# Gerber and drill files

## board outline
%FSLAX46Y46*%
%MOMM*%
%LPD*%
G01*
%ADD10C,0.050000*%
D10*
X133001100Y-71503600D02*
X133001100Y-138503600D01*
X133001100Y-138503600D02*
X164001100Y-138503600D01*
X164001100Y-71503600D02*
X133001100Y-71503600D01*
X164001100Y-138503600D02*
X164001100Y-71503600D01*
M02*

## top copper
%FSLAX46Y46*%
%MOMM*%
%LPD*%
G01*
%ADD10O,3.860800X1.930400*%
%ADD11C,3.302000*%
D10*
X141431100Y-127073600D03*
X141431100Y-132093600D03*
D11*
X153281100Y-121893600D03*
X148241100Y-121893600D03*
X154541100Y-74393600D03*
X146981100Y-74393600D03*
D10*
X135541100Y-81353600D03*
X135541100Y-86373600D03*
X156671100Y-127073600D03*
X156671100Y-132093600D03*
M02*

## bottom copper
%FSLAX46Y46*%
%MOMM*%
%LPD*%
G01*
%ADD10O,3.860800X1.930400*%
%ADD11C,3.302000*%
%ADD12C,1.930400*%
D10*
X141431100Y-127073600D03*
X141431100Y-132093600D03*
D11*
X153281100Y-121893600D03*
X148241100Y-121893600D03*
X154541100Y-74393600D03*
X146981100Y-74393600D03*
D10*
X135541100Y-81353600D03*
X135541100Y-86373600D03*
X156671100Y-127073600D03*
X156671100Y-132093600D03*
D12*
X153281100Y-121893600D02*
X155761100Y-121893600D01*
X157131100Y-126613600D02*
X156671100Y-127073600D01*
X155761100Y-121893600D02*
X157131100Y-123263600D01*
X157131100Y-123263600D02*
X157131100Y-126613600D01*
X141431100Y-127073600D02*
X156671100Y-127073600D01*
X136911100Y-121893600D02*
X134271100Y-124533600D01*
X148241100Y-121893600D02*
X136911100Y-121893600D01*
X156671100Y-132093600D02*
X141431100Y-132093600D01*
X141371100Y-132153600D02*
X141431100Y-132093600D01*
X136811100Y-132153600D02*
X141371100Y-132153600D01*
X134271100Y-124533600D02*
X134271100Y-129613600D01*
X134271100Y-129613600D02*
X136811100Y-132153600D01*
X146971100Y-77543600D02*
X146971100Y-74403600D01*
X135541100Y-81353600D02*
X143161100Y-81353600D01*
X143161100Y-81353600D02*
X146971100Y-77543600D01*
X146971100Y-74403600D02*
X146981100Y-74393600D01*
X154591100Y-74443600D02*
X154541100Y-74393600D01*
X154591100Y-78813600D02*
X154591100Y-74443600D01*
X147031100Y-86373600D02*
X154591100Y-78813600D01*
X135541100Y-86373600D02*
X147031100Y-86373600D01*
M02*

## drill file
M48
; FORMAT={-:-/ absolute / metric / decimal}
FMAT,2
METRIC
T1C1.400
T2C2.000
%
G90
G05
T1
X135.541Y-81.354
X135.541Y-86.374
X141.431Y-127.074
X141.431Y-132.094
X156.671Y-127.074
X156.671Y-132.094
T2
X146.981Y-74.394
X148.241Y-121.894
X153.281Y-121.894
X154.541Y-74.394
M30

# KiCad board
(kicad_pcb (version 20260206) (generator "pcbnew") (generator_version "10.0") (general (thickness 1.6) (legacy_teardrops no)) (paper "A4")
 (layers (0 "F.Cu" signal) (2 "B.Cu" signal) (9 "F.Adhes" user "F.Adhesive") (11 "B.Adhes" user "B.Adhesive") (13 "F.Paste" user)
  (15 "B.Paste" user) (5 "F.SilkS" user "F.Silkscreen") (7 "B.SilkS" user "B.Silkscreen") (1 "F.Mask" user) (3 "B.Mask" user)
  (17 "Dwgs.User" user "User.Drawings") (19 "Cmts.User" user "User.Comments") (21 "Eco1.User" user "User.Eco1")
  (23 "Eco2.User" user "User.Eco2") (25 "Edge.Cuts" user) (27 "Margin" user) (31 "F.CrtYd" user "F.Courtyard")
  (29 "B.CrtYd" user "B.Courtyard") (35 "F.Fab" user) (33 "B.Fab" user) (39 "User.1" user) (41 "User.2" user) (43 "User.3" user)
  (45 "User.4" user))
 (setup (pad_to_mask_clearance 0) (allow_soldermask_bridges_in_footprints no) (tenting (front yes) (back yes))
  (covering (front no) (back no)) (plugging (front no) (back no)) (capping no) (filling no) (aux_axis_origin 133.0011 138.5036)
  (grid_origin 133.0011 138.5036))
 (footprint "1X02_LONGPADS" (layer "F.Cu") (at 141.4311 127.0736 -90)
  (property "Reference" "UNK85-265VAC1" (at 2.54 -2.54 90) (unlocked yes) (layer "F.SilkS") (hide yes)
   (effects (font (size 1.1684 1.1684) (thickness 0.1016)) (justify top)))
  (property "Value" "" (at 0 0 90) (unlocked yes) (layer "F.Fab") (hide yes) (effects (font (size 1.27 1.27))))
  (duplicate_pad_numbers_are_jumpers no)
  (pad "1" thru_hole oval (at 0 0) (size 3.8608 1.9304) (drill 1.4) (layers "*.Cu" "*.Mask") (remove_unused_layers no) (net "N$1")
   (solder_mask_margin 0.1016) (thermal_bridge_angle 0))
  (pad "2" thru_hole oval (at 5.02 0) (size 3.8608 1.9304) (drill 1.4) (layers "*.Cu" "*.Mask") (remove_unused_layers no) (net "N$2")
   (solder_mask_margin 0.1016) (thermal_bridge_angle 0)))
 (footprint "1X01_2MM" (layer "F.Cu") (at 153.2811 121.8936)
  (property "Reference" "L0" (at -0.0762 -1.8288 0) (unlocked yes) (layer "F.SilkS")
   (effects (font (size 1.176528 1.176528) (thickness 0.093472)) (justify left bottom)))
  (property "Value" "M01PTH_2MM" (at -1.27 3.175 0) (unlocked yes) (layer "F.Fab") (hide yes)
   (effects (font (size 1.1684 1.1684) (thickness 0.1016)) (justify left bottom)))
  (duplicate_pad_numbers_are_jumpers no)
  (pad "1" thru_hole circle (at 0 0 90) (size 3.302 3.302) (drill 2) (layers "*.Cu" "*.Mask") (remove_unused_layers no) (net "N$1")
   (solder_mask_margin 0.1016) (thermal_bridge_angle 0)))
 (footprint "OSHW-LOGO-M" (layer "F.Cu") (at 135.5411 75.0036 90)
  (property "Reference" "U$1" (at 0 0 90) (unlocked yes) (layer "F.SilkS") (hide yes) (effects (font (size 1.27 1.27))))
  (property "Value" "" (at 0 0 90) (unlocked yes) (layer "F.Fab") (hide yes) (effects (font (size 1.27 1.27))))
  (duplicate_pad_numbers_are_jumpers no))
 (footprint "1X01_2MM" (layer "F.Cu") (at 148.2411 121.8936)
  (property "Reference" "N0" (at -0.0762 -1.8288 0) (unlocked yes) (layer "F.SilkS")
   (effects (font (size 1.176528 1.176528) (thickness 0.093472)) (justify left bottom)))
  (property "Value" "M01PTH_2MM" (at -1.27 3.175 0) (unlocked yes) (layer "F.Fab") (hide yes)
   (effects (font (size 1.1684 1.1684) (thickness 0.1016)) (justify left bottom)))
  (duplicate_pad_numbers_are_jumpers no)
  (pad "1" thru_hole circle (at 0 0 90) (size 3.302 3.302) (drill 2) (layers "*.Cu" "*.Mask") (remove_unused_layers no) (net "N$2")
   (solder_mask_margin 0.1016) (thermal_bridge_angle 0)))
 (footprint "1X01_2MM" (layer "F.Cu") (at 154.5411 74.3936)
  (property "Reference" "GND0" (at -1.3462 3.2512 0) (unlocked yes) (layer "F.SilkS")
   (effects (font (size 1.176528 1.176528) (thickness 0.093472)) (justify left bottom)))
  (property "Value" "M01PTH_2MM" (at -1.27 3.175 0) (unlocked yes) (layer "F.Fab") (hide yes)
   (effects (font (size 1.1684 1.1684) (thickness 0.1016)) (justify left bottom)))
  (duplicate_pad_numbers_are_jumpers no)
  (pad "1" thru_hole circle (at 0 0 90) (size 3.302 3.302) (drill 2) (layers "*.Cu" "*.Mask") (remove_unused_layers no) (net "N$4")
   (solder_mask_margin 0.1016) (thermal_bridge_angle 0)))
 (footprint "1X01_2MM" (layer "F.Cu") (at 146.9811 74.3936)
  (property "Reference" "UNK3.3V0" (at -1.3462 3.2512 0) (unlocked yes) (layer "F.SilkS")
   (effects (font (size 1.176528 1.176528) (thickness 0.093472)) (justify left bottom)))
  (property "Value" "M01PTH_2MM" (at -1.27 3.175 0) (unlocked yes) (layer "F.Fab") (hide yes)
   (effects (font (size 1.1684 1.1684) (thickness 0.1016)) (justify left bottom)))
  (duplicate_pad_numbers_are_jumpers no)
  (pad "1" thru_hole circle (at 0 0 90) (size 3.302 3.302) (drill 2) (layers "*.Cu" "*.Mask") (remove_unused_layers no) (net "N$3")
   (solder_mask_margin 0.1016) (thermal_bridge_angle 0)))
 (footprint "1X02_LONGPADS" (layer "F.Cu") (at 135.5411 81.3536 -90)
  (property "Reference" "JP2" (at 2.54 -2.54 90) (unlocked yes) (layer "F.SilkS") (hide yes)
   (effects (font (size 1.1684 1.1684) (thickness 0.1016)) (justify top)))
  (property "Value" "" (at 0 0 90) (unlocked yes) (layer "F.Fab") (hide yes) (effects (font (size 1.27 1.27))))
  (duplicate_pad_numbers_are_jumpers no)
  (pad "1" thru_hole oval (at 0 0) (size 3.8608 1.9304) (drill 1.4) (layers "*.Cu" "*.Mask") (remove_unused_layers no) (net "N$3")
   (solder_mask_margin 0.1016) (thermal_bridge_angle 0))
  (pad "2" thru_hole oval (at 5.02 0) (size 3.8608 1.9304) (drill 1.4) (layers "*.Cu" "*.Mask") (remove_unused_layers no) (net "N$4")
   (solder_mask_margin 0.1016) (thermal_bridge_angle 0)))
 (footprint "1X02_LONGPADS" (layer "F.Cu") (at 156.6711 127.0736 -90)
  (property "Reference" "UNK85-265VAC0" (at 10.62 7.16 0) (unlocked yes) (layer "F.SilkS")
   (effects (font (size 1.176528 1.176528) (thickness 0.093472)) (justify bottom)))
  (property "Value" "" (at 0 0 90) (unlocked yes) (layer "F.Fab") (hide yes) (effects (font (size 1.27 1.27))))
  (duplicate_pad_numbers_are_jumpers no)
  (pad "1" thru_hole oval (at 0 0) (size 3.8608 1.9304) (drill 1.4) (layers "*.Cu" "*.Mask") (remove_unused_layers no) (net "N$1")
   (solder_mask_margin 0.1016) (thermal_bridge_angle 0))
  (pad "2" thru_hole oval (at 5.02 0) (size 3.8608 1.9304) (drill 1.4) (layers "*.Cu" "*.Mask") (remove_unused_layers no) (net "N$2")
   (solder_mask_margin 0.1016) (thermal_bridge_angle 0)))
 (gr_line (start 133.0011 71.5036) (end 133.0011 138.5036) (stroke (width 0.05) (type solid)) (layer "Edge.Cuts"))
 (gr_line (start 133.0011 138.5036) (end 164.0011 138.5036) (stroke (width 0.05) (type solid)) (layer "Edge.Cuts"))
 (gr_line (start 164.0011 71.5036) (end 133.0011 71.5036) (stroke (width 0.05) (type solid)) (layer "Edge.Cuts"))
 (gr_line (start 164.0011 138.5036) (end 164.0011 71.5036) (stroke (width 0.05) (type solid)) (layer "Edge.Cuts"))
 (segment (start 153.2811 121.8936) (end 155.7611 121.8936) (width 1.9304) (layer "B.Cu") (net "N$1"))
 (segment (start 157.1311 126.6136) (end 156.6711 127.0736) (width 1.9304) (layer "B.Cu") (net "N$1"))
 (segment (start 155.7611 121.8936) (end 157.1311 123.2636) (width 1.9304) (layer "B.Cu") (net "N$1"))
 (segment (start 157.1311 123.2636) (end 157.1311 126.6136) (width 1.9304) (layer "B.Cu") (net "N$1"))
 (segment (start 141.4311 127.0736) (end 156.6711 127.0736) (width 1.9304) (layer "B.Cu") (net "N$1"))
 (segment (start 136.9111 121.8936) (end 134.2711 124.5336) (width 1.9304) (layer "B.Cu") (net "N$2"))
 (segment (start 148.2411 121.8936) (end 136.9111 121.8936) (width 1.9304) (layer "B.Cu") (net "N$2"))
 (segment (start 156.6711 132.0936) (end 141.4311 132.0936) (width 1.9304) (layer "B.Cu") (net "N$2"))
 (segment (start 141.3711 132.1536) (end 141.4311 132.0936) (width 1.9304) (layer "B.Cu") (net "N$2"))
 (segment (start 136.8111 132.1536) (end 141.3711 132.1536) (width 1.9304) (layer "B.Cu") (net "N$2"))
 (segment (start 134.2711 124.5336) (end 134.2711 129.6136) (width 1.9304) (layer "B.Cu") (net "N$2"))
 (segment (start 134.2711 129.6136) (end 136.8111 132.1536) (width 1.9304) (layer "B.Cu") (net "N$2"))
 (segment (start 146.9711 77.5436) (end 146.9711 74.4036) (width 1.9304) (layer "B.Cu") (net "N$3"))
 (segment (start 135.5411 81.3536) (end 143.1611 81.3536) (width 1.9304) (layer "B.Cu") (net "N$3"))
 (segment (start 143.1611 81.3536) (end 146.9711 77.5436) (width 1.9304) (layer "B.Cu") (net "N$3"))
 (segment (start 146.9711 74.4036) (end 146.9811 74.3936) (width 1.9304) (layer "B.Cu") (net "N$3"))
 (segment (start 154.5911 74.4436) (end 154.5411 74.3936) (width 1.9304) (layer "B.Cu") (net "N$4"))
 (segment (start 154.5911 78.8136) (end 154.5911 74.4436) (width 1.9304) (layer "B.Cu") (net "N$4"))
 (segment (start 147.0311 86.3736) (end 154.5911 78.8136) (width 1.9304) (layer "B.Cu") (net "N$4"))
 (segment (start 135.5411 86.3736) (end 147.0311 86.3736) (width 1.9304) (layer "B.Cu") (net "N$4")))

